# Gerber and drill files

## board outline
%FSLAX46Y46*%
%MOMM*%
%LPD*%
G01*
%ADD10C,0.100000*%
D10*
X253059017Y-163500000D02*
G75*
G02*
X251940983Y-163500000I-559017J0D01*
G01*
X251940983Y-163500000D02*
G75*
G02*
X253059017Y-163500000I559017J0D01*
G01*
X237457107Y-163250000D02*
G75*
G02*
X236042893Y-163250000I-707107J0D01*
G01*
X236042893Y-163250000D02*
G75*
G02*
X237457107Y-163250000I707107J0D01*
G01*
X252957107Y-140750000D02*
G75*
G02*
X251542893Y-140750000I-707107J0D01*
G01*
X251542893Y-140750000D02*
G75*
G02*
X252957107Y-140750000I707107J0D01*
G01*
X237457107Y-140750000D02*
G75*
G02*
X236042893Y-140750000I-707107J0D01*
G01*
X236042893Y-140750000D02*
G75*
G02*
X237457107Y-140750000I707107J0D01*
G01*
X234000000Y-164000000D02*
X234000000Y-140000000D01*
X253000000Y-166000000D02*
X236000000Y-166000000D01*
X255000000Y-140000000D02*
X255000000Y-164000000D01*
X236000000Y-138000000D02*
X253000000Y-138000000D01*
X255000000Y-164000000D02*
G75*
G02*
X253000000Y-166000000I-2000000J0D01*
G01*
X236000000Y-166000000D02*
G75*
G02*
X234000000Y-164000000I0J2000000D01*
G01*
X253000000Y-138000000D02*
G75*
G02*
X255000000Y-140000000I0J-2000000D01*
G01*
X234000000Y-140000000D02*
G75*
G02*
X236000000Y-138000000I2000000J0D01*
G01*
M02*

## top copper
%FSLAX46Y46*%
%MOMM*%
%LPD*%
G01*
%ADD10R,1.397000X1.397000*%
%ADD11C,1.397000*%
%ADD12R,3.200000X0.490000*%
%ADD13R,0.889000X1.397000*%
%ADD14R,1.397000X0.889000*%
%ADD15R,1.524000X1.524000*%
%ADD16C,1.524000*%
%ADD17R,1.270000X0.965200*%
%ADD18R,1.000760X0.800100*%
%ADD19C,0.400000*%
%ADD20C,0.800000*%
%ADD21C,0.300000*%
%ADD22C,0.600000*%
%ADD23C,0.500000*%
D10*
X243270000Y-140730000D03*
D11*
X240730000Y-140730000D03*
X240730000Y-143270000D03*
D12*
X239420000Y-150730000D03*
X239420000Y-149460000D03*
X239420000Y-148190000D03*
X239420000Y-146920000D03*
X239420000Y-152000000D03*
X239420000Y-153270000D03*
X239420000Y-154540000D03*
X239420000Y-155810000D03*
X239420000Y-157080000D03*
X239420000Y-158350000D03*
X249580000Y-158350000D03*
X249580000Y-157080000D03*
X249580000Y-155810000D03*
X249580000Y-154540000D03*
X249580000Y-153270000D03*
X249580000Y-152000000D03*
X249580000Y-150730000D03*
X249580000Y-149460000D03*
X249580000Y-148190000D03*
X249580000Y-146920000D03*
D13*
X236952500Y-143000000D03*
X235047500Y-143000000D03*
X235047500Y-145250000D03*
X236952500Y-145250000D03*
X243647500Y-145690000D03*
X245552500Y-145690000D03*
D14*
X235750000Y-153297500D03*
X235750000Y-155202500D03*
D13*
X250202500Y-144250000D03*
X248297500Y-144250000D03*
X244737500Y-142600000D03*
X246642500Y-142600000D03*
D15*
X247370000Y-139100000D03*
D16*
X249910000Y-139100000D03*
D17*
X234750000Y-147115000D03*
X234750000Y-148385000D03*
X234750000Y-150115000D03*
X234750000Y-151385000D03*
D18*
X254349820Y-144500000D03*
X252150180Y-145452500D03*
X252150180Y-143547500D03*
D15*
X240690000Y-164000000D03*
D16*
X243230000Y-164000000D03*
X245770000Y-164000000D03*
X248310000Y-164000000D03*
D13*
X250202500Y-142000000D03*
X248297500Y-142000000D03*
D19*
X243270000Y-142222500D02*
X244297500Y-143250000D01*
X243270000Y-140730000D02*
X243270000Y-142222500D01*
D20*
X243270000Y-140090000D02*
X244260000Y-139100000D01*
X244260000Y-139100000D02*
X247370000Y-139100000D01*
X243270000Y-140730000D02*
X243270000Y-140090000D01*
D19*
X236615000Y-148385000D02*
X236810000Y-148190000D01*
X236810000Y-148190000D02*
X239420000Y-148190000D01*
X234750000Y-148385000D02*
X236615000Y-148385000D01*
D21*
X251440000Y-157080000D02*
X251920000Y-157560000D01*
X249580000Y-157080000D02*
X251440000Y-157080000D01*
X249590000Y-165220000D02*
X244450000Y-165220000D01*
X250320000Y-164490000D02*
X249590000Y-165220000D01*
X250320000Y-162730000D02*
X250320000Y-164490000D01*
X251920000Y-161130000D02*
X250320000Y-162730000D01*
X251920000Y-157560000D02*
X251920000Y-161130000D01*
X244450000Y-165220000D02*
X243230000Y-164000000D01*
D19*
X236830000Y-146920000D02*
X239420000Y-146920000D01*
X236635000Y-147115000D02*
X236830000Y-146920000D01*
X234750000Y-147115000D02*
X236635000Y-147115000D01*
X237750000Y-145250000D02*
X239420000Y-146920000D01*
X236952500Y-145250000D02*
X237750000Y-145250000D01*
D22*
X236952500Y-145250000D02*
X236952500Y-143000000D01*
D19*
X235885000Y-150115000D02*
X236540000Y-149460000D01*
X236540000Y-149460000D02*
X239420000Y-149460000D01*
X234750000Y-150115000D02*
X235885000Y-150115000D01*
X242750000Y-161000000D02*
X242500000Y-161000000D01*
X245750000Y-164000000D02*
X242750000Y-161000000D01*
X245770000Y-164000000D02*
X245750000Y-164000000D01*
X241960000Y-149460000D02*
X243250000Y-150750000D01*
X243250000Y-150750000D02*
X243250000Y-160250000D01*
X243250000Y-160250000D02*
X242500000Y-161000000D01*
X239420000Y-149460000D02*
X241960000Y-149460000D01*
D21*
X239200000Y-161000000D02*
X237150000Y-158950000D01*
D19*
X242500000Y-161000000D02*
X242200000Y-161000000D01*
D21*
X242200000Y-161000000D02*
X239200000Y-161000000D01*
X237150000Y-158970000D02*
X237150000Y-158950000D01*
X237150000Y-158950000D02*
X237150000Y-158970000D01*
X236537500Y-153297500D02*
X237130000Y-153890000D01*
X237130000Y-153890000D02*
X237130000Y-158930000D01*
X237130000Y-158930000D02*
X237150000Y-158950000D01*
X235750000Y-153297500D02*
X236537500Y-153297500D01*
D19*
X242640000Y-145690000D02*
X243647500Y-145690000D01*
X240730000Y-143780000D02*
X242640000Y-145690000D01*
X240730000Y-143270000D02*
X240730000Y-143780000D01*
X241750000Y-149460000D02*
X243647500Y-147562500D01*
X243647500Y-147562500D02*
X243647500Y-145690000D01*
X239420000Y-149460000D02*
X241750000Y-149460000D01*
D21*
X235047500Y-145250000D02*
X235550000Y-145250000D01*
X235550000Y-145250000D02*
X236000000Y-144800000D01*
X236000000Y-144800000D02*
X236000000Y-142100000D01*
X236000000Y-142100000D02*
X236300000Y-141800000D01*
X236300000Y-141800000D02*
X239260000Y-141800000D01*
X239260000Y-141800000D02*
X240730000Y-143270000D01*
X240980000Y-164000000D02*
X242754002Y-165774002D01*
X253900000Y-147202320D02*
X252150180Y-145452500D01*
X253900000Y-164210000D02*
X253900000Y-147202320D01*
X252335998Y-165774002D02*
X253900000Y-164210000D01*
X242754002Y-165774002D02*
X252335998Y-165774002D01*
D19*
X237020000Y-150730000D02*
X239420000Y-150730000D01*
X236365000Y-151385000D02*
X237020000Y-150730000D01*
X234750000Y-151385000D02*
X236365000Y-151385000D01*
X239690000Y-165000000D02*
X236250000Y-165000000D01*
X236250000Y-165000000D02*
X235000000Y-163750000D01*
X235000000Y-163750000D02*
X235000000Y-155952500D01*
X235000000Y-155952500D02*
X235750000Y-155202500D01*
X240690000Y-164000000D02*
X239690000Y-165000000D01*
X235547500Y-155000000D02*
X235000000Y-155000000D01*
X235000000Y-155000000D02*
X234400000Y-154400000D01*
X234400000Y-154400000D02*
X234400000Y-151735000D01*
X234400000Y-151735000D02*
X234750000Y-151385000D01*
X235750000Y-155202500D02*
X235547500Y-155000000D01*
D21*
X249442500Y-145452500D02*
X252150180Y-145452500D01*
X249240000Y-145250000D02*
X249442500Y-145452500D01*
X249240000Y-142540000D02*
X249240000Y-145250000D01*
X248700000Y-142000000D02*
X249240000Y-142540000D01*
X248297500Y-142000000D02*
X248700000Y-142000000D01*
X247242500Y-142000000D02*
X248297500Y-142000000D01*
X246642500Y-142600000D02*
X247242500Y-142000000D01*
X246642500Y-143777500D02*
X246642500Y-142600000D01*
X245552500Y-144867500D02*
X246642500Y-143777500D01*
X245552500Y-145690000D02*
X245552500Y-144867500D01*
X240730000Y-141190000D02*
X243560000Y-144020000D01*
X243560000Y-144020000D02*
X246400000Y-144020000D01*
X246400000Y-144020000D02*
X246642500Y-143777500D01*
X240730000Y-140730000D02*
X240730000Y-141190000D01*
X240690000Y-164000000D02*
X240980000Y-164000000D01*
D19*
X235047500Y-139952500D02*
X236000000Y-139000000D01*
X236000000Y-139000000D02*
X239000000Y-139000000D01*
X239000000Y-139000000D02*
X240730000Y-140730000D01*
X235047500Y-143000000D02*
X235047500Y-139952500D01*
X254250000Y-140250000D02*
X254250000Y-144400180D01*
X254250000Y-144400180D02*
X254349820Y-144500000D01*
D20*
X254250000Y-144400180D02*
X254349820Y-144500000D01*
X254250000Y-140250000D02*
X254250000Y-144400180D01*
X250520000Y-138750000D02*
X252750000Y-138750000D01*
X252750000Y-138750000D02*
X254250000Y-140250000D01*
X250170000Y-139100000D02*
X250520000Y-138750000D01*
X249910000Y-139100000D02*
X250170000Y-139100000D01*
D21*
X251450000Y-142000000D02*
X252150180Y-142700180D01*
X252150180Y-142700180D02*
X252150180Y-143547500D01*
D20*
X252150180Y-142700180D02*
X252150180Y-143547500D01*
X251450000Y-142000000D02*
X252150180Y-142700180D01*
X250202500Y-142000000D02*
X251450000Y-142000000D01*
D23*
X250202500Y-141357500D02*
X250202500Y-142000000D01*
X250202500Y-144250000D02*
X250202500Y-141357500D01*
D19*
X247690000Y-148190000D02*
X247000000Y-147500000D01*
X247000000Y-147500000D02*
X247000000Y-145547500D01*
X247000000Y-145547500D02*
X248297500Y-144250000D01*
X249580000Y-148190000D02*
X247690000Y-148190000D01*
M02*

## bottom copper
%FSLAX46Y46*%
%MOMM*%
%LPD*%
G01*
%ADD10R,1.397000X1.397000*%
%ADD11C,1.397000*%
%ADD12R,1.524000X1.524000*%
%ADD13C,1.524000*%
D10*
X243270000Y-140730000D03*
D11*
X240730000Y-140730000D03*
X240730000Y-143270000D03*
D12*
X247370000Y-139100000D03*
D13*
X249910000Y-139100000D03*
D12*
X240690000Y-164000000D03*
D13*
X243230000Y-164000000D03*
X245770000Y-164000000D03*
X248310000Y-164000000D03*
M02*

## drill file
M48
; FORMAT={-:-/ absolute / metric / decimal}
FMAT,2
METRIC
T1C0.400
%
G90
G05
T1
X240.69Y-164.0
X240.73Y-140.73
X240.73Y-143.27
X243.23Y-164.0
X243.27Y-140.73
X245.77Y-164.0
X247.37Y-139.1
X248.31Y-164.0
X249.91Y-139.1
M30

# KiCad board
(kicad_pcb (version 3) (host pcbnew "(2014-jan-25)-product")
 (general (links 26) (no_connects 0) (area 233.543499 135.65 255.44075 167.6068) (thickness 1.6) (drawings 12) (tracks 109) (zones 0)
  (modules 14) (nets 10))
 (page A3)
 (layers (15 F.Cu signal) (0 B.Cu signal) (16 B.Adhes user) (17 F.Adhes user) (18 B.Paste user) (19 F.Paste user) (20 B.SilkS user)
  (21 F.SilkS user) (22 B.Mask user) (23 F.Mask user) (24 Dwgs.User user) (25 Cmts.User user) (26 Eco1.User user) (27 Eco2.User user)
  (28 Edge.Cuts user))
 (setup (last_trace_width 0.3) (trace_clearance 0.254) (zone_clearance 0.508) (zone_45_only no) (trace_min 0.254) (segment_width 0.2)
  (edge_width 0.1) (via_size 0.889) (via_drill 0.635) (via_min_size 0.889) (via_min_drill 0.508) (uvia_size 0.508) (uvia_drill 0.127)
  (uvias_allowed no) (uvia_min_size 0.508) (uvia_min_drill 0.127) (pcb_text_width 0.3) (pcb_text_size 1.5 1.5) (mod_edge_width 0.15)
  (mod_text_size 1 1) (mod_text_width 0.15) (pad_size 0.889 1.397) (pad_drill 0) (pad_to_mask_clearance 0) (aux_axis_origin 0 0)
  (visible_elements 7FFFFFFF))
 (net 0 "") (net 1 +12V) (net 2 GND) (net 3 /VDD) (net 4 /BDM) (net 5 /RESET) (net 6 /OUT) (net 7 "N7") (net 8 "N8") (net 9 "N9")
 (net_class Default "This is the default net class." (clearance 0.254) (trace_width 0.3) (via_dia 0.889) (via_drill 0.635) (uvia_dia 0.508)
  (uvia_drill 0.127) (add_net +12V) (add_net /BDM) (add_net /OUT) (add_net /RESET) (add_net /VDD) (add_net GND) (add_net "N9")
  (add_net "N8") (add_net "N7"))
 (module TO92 (layer F.Cu) (at 242 142)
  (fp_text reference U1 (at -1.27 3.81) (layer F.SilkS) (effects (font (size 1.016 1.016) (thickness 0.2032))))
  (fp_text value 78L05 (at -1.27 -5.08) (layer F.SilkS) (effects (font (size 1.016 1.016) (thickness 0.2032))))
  (pad 1 thru_hole rect (at 1.27 -1.27) (size 1.397 1.397) (drill 0.4) (layers *.Cu *.Mask F.SilkS) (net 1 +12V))
  (pad 2 thru_hole circle (at -1.27 -1.27) (size 1.397 1.397) (drill 0.4) (layers *.Cu *.Mask F.SilkS) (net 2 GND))
  (pad 3 thru_hole circle (at -1.27 1.27) (size 1.397 1.397) (drill 0.4) (layers *.Cu *.Mask F.SilkS) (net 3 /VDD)))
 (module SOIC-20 (layer F.Cu) (at 244.5 152)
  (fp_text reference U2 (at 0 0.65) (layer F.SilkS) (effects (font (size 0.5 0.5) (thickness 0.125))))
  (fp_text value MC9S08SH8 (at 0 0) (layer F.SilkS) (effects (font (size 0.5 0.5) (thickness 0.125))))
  (pad 4 smd rect (at -5.08 -1.27) (size 3.2 0.49) (layers F.Cu F.Paste F.Mask) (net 2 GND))
  (pad 3 smd rect (at -5.08 -2.54) (size 3.2 0.49) (layers F.Cu F.Paste F.Mask) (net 3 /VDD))
  (pad 2 smd rect (at -5.08 -3.81) (size 3.2 0.49) (layers F.Cu F.Paste F.Mask) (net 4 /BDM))
  (pad 1 smd rect (at -5.08 -5.08) (size 3.2 0.49) (layers F.Cu F.Paste F.Mask) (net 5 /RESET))
  (pad 5 smd rect (at -5.08 0) (size 3.2 0.49) (layers F.Cu F.Paste F.Mask))
  (pad 6 smd rect (at -5.08 1.27) (size 3.2 0.49) (layers F.Cu F.Paste F.Mask))
  (pad 7 smd rect (at -5.08 2.54) (size 3.2 0.49) (layers F.Cu F.Paste F.Mask))
  (pad 8 smd rect (at -5.08 3.81) (size 3.2 0.49) (layers F.Cu F.Paste F.Mask))
  (pad 9 smd rect (at -5.08 5.08) (size 3.2 0.49) (layers F.Cu F.Paste F.Mask))
  (pad 10 smd rect (at -5.08 6.35) (size 3.2 0.49) (layers F.Cu F.Paste F.Mask))
  (pad 11 smd rect (at 5.08 6.35) (size 3.2 0.49) (layers F.Cu F.Paste F.Mask))
  (pad 12 smd rect (at 5.08 5.08) (size 3.2 0.49) (layers F.Cu F.Paste F.Mask) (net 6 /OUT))
  (pad 13 smd rect (at 5.08 3.81) (size 3.2 0.49) (layers F.Cu F.Paste F.Mask))
  (pad 14 smd rect (at 5.08 2.54) (size 3.2 0.49) (layers F.Cu F.Paste F.Mask))
  (pad 15 smd rect (at 5.08 1.27) (size 3.2 0.49) (layers F.Cu F.Paste F.Mask))
  (pad 16 smd rect (at 5.08 0) (size 3.2 0.49) (layers F.Cu F.Paste F.Mask))
  (pad 17 smd rect (at 5.08 -1.27) (size 3.2 0.49) (layers F.Cu F.Paste F.Mask))
  (pad 18 smd rect (at 5.08 -2.54) (size 3.2 0.49) (layers F.Cu F.Paste F.Mask))
  (pad 19 smd rect (at 5.08 -3.81) (size 3.2 0.49) (layers F.Cu F.Paste F.Mask) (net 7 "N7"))
  (pad 20 smd rect (at 5.08 -5.08) (size 3.2 0.49) (layers F.Cu F.Paste F.Mask)))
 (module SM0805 (layer F.Cu) (at 236 143 180)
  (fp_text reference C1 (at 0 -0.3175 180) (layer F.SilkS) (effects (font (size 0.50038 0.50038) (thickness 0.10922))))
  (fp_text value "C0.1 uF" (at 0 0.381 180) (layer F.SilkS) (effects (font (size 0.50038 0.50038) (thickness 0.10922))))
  (pad 1 smd rect (at -0.9525 0 180) (size 0.889 1.397) (layers F.Cu F.Paste F.Mask) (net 5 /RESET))
  (pad 2 smd rect (at 0.9525 0 180) (size 0.889 1.397) (layers F.Cu F.Paste F.Mask) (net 2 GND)))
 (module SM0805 (layer F.Cu) (at 236 145.25)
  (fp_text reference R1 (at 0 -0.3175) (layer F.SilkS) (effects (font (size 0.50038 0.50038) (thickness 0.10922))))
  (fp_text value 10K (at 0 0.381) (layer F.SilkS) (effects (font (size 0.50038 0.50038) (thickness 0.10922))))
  (pad 1 smd rect (at -0.9525 0) (size 0.889 1.397) (layers F.Cu F.Paste F.Mask) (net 3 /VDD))
  (pad 2 smd rect (at 0.9525 0) (size 0.889 1.397) (layers F.Cu F.Paste F.Mask) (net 5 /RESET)))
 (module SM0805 (layer F.Cu) (at 244.6 145.69)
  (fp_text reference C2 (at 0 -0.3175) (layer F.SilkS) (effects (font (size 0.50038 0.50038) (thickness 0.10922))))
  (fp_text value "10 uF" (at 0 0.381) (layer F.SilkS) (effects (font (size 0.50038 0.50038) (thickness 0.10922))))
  (pad 1 smd rect (at -0.9525 0) (size 0.889 1.397) (layers F.Cu F.Paste F.Mask) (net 3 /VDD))
  (pad 2 smd rect (at 0.9525 0) (size 0.889 1.397) (layers F.Cu F.Paste F.Mask) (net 2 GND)))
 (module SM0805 (layer F.Cu) (at 235.75 154.25 270)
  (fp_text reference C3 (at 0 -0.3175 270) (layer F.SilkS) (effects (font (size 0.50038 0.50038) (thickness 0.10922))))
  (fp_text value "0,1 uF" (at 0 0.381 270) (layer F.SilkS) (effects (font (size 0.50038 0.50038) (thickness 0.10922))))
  (pad 1 smd rect (at -0.9525 0 270) (size 0.889 1.397) (layers F.Cu F.Paste F.Mask) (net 3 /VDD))
  (pad 2 smd rect (at 0.9525 0 270) (size 0.889 1.397) (layers F.Cu F.Paste F.Mask) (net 2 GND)))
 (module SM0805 (layer F.Cu) (at 249.25 144.25 180)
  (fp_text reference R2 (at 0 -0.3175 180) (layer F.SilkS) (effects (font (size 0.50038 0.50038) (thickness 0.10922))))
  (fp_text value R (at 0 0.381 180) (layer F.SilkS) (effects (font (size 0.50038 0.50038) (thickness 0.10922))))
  (pad 1 smd rect (at -0.9525 0 180) (size 0.889 1.397) (layers F.Cu F.Paste F.Mask) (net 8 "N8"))
  (pad 2 smd rect (at 0.9525 0 180) (size 0.889 1.397) (layers F.Cu F.Paste F.Mask) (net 7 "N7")))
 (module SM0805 (layer F.Cu) (at 245.69 142.6)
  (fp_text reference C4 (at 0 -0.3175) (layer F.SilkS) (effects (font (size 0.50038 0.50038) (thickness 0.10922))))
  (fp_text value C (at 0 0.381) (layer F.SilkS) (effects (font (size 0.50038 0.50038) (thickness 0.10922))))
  (pad 1 smd rect (at -0.9525 0) (size 0.889 1.397) (layers F.Cu F.Paste F.Mask) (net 1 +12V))
  (pad 2 smd rect (at 0.9525 0) (size 0.889 1.397) (layers F.Cu F.Paste F.Mask) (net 2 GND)))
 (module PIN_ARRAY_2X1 (layer F.Cu) (at 248.64 139.1)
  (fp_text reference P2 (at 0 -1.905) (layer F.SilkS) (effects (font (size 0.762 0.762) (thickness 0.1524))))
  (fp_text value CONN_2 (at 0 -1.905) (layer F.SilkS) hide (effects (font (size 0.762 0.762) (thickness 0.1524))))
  (pad 1 thru_hole rect (at -1.27 0) (size 1.524 1.524) (drill 0.4) (layers *.Cu *.Mask F.SilkS) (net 1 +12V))
  (pad 2 thru_hole circle (at 1.27 0) (size 1.524 1.524) (drill 0.4) (layers *.Cu *.Mask F.SilkS) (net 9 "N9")))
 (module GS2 (layer F.Cu) (at 234.75 147.75)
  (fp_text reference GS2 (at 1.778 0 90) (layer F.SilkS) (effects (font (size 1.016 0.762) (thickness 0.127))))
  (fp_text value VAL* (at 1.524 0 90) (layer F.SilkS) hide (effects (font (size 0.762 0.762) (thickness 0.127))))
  (pad 1 smd rect (at 0 -0.635) (size 1.27 0.9652) (layers F.Cu F.Paste F.Mask) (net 5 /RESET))
  (pad 2 smd rect (at 0 0.635) (size 1.27 0.9652) (layers F.Cu F.Paste F.Mask) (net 4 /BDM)))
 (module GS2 (layer F.Cu) (at 234.75 150.75)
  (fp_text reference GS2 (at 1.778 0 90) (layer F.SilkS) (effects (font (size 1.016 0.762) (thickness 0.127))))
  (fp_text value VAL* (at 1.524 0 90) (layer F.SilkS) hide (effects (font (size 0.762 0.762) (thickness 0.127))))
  (pad 1 smd rect (at 0 -0.635) (size 1.27 0.9652) (layers F.Cu F.Paste F.Mask) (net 3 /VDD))
  (pad 2 smd rect (at 0 0.635) (size 1.27 0.9652) (layers F.Cu F.Paste F.Mask) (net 2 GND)))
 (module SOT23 (layer F.Cu) (at 253.25 144.5 270)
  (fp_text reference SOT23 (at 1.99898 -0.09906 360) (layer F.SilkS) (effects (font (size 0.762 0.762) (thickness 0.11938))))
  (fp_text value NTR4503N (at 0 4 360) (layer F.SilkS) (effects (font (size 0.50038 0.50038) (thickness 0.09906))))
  (pad 3 smd rect (at 0 -1.09982 270) (size 0.8001 1.00076) (layers F.Cu F.Paste F.Mask) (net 9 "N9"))
  (pad 2 smd rect (at 0.9525 1.09982 270) (size 0.8001 1.00076) (layers F.Cu F.Paste F.Mask) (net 2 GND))
  (pad 1 smd rect (at -0.9525 1.09982 270) (size 0.8001 1.00076) (layers F.Cu F.Paste F.Mask) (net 8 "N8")))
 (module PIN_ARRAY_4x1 (layer F.Cu) (at 244.5 164)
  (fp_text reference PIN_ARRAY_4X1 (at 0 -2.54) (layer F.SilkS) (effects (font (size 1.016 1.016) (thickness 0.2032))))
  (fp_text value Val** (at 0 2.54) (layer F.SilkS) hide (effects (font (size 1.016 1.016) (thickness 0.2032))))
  (pad 1 thru_hole rect (at -3.81 0) (size 1.524 1.524) (drill 0.4) (layers *.Cu *.Mask F.SilkS) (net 2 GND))
  (pad 2 thru_hole circle (at -1.27 0) (size 1.524 1.524) (drill 0.4) (layers *.Cu *.Mask F.SilkS) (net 6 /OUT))
  (pad 3 thru_hole circle (at 1.27 0) (size 1.524 1.524) (drill 0.4) (layers *.Cu *.Mask F.SilkS) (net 3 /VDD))
  (pad 4 thru_hole circle (at 3.81 0) (size 1.524 1.524) (drill 0.4) (layers *.Cu *.Mask F.SilkS)))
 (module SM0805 (layer F.Cu) (at 249.25 142 180)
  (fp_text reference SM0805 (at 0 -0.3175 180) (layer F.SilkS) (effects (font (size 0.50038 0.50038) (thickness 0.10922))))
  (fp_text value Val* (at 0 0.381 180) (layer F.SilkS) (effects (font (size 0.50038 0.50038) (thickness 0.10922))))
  (pad 1 smd rect (at -0.9525 0 180) (size 0.889 1.397) (layers F.Cu F.Paste F.Mask) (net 8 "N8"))
  (pad 2 smd rect (at 0.9525 0 180) (size 0.889 1.397) (layers F.Cu F.Paste F.Mask) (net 2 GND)))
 (gr_circle (center 252.5 163.5) (end 253 163.75) (layer Edge.Cuts) (width 0.1))
 (gr_circle (center 236.75 163.25) (end 237.25 163.75) (layer Edge.Cuts) (width 0.1))
 (gr_circle (center 252.25 140.75) (end 252.75 140.25) (layer Edge.Cuts) (width 0.1))
 (gr_circle (center 236.75 140.75) (end 236.25 140.25) (layer Edge.Cuts) (width 0.1))
 (gr_line (start 234 164) (end 234 140) (angle 90) (layer Edge.Cuts) (width 0.1))
 (gr_line (start 253 166) (end 236 166) (angle 90) (layer Edge.Cuts) (width 0.1))
 (gr_line (start 255 140) (end 255 164) (angle 90) (layer Edge.Cuts) (width 0.1))
 (gr_line (start 236 138) (end 253 138) (angle 90) (layer Edge.Cuts) (width 0.1))
 (gr_arc (start 253 164) (end 255 164) (angle 90) (layer Edge.Cuts) (width 0.1))
 (gr_arc (start 236 164) (end 236 166) (angle 90) (layer Edge.Cuts) (width 0.1))
 (gr_arc (start 253 140) (end 253 138) (angle 90) (layer Edge.Cuts) (width 0.1))
 (gr_arc (start 236 140) (end 234 140) (angle 90) (layer Edge.Cuts) (width 0.1))
 (segment (start 243.27 142.2225) (end 244.2975 143.25) (width 0.4) (layer F.Cu) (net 1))
 (segment (start 243.27 140.73) (end 243.27 142.2225) (width 0.4) (layer F.Cu) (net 1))
 (segment (start 243.27 140.09) (end 244.26 139.1) (width 0.8) (layer F.Cu) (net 1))
 (segment (start 244.26 139.1) (end 247.37 139.1) (width 0.8) (layer F.Cu) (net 1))
 (segment (start 243.27 140.73) (end 243.27 140.09) (width 0.8) (layer F.Cu) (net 1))
 (segment (start 236.615 148.385) (end 236.81 148.19) (width 0.4) (layer F.Cu) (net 4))
 (segment (start 236.81 148.19) (end 239.42 148.19) (width 0.4) (layer F.Cu) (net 4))
 (segment (start 234.75 148.385) (end 236.615 148.385) (width 0.4) (layer F.Cu) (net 4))
 (segment (start 251.44 157.08) (end 251.92 157.56) (width 0.3) (layer F.Cu) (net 6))
 (segment (start 249.58 157.08) (end 251.44 157.08) (width 0.3) (layer F.Cu) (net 6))
 (segment (start 249.59 165.22) (end 244.45 165.22) (width 0.3) (layer F.Cu) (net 6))
 (segment (start 250.32 164.49) (end 249.59 165.22) (width 0.3) (layer F.Cu) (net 6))
 (segment (start 250.32 162.73) (end 250.32 164.49) (width 0.3) (layer F.Cu) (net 6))
 (segment (start 251.92 161.13) (end 250.32 162.73) (width 0.3) (layer F.Cu) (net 6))
 (segment (start 251.92 157.56) (end 251.92 161.13) (width 0.3) (layer F.Cu) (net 6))
 (segment (start 244.45 165.22) (end 243.23 164) (width 0.3) (layer F.Cu) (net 6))
 (segment (start 236.83 146.92) (end 239.42 146.92) (width 0.4) (layer F.Cu) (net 5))
 (segment (start 236.635 147.115) (end 236.83 146.92) (width 0.4) (layer F.Cu) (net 5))
 (segment (start 234.75 147.115) (end 236.635 147.115) (width 0.4) (layer F.Cu) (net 5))
 (segment (start 237.75 145.25) (end 239.42 146.92) (width 0.4) (layer F.Cu) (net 5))
 (segment (start 236.9525 145.25) (end 237.75 145.25) (width 0.4) (layer F.Cu) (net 5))
 (segment (start 236.9525 145.25) (end 236.9525 143) (width 0.6) (layer F.Cu) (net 5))
 (segment (start 235.885 150.115) (end 236.54 149.46) (width 0.4) (layer F.Cu) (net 3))
 (segment (start 236.54 149.46) (end 239.42 149.46) (width 0.4) (layer F.Cu) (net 3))
 (segment (start 234.75 150.115) (end 235.885 150.115) (width 0.4) (layer F.Cu) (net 3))
 (segment (start 242.75 161) (end 242.5 161) (width 0.4) (layer F.Cu) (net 3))
 (segment (start 245.75 164) (end 242.75 161) (width 0.4) (layer F.Cu) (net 3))
 (segment (start 245.77 164) (end 245.75 164) (width 0.4) (layer F.Cu) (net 3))
 (segment (start 241.96 149.46) (end 243.25 150.75) (width 0.4) (layer F.Cu) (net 3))
 (segment (start 243.25 150.75) (end 243.25 160.25) (width 0.4) (layer F.Cu) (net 3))
 (segment (start 243.25 160.25) (end 242.5 161) (width 0.4) (layer F.Cu) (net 3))
 (segment (start 239.42 149.46) (end 241.96 149.46) (width 0.4) (layer F.Cu) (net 3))
 (segment (start 239.2 161) (end 237.15 158.95) (width 0.3) (layer F.Cu) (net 3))
 (segment (start 242.5 161) (end 242.2 161) (width 0.4) (layer F.Cu) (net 3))
 (segment (start 242.2 161) (end 239.2 161) (width 0.3) (layer F.Cu) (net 3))
 (segment (start 237.15 158.97) (end 237.15 158.95) (width 0.3) (layer F.Cu) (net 3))
 (segment (start 237.15 158.95) (end 237.15 158.97) (width 0.3) (layer F.Cu) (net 3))
 (segment (start 236.5375 153.2975) (end 237.13 153.89) (width 0.3) (layer F.Cu) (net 3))
 (segment (start 237.13 153.89) (end 237.13 158.93) (width 0.3) (layer F.Cu) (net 3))
 (segment (start 237.13 158.93) (end 237.15 158.95) (width 0.3) (layer F.Cu) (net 3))
 (segment (start 235.75 153.2975) (end 236.5375 153.2975) (width 0.3) (layer F.Cu) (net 3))
 (segment (start 242.64 145.69) (end 243.6475 145.69) (width 0.4) (layer F.Cu) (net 3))
 (segment (start 240.73 143.78) (end 242.64 145.69) (width 0.4) (layer F.Cu) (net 3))
 (segment (start 240.73 143.27) (end 240.73 143.78) (width 0.4) (layer F.Cu) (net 3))
 (segment (start 241.75 149.46) (end 243.6475 147.5625) (width 0.4) (layer F.Cu) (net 3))
 (segment (start 243.6475 147.5625) (end 243.6475 145.69) (width 0.4) (layer F.Cu) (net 3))
 (segment (start 239.42 149.46) (end 241.75 149.46) (width 0.4) (layer F.Cu) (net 3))
 (segment (start 235.0475 145.25) (end 235.55 145.25) (width 0.3) (layer F.Cu) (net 3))
 (segment (start 235.55 145.25) (end 236 144.8) (width 0.3) (layer F.Cu) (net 3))
 (segment (start 236 144.8) (end 236 142.1) (width 0.3) (layer F.Cu) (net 3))
 (segment (start 236 142.1) (end 236.3 141.8) (width 0.3) (layer F.Cu) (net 3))
 (segment (start 236.3 141.8) (end 239.26 141.8) (width 0.3) (layer F.Cu) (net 3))
 (segment (start 239.26 141.8) (end 240.73 143.27) (width 0.3) (layer F.Cu) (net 3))
 (segment (start 240.98 164) (end 242.754002 165.774002) (width 0.3) (layer F.Cu) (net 2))
 (segment (start 253.9 147.20232) (end 252.15018 145.4525) (width 0.3) (layer F.Cu) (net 2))
 (segment (start 253.9 164.21) (end 253.9 147.20232) (width 0.3) (layer F.Cu) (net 2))
 (segment (start 252.335998 165.774002) (end 253.9 164.21) (width 0.3) (layer F.Cu) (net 2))
 (segment (start 242.754002 165.774002) (end 252.335998 165.774002) (width 0.3) (layer F.Cu) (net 2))
 (segment (start 237.02 150.73) (end 239.42 150.73) (width 0.4) (layer F.Cu) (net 2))
 (segment (start 236.365 151.385) (end 237.02 150.73) (width 0.4) (layer F.Cu) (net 2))
 (segment (start 234.75 151.385) (end 236.365 151.385) (width 0.4) (layer F.Cu) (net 2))
 (segment (start 239.69 165) (end 236.25 165) (width 0.4) (layer F.Cu) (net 2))
 (segment (start 236.25 165) (end 235 163.75) (width 0.4) (layer F.Cu) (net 2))
 (segment (start 235 163.75) (end 235 155.9525) (width 0.4) (layer F.Cu) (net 2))
 (segment (start 235 155.9525) (end 235.75 155.2025) (width 0.4) (layer F.Cu) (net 2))
 (segment (start 240.69 164) (end 239.69 165) (width 0.4) (layer F.Cu) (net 2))
 (segment (start 235.5475 155) (end 235 155) (width 0.4) (layer F.Cu) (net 2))
 (segment (start 235 155) (end 234.4 154.4) (width 0.4) (layer F.Cu) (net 2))
 (segment (start 234.4 154.4) (end 234.4 151.735) (width 0.4) (layer F.Cu) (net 2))
 (segment (start 234.4 151.735) (end 234.75 151.385) (width 0.4) (layer F.Cu) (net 2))
 (segment (start 235.75 155.2025) (end 235.5475 155) (width 0.4) (layer F.Cu) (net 2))
 (segment (start 249.4425 145.4525) (end 252.15018 145.4525) (width 0.3) (layer F.Cu) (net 2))
 (segment (start 249.24 145.25) (end 249.4425 145.4525) (width 0.3) (layer F.Cu) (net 2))
 (segment (start 249.24 142.54) (end 249.24 145.25) (width 0.3) (layer F.Cu) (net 2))
 (segment (start 248.7 142) (end 249.24 142.54) (width 0.3) (layer F.Cu) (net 2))
 (segment (start 248.2975 142) (end 248.7 142) (width 0.3) (layer F.Cu) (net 2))
 (segment (start 247.2425 142) (end 248.2975 142) (width 0.3) (layer F.Cu) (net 2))
 (segment (start 246.6425 142.6) (end 247.2425 142) (width 0.3) (layer F.Cu) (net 2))
 (segment (start 246.6425 143.7775) (end 246.6425 142.6) (width 0.3) (layer F.Cu) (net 2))
 (segment (start 245.5525 144.8675) (end 246.6425 143.7775) (width 0.3) (layer F.Cu) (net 2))
 (segment (start 245.5525 145.69) (end 245.5525 144.8675) (width 0.3) (layer F.Cu) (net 2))
 (segment (start 240.73 141.19) (end 243.56 144.02) (width 0.3) (layer F.Cu) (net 2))
 (segment (start 243.56 144.02) (end 246.4 144.02) (width 0.3) (layer F.Cu) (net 2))
 (segment (start 246.4 144.02) (end 246.6425 143.7775) (width 0.3) (layer F.Cu) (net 2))
 (segment (start 240.73 140.73) (end 240.73 141.19) (width 0.3) (layer F.Cu) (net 2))
 (segment (start 240.69 164) (end 240.98 164) (width 0.3) (layer F.Cu) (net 2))
 (segment (start 235.0475 139.9525) (end 236 139) (width 0.4) (layer F.Cu) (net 2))
 (segment (start 236 139) (end 239 139) (width 0.4) (layer F.Cu) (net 2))
 (segment (start 239 139) (end 240.73 140.73) (width 0.4) (layer F.Cu) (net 2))
 (segment (start 235.0475 143) (end 235.0475 139.9525) (width 0.4) (layer F.Cu) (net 2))
 (segment (start 254.25 140.25) (end 254.25 144.40018) (width 0.4) (layer F.Cu) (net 9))
 (segment (start 254.25 144.40018) (end 254.34982 144.5) (width 0.4) (layer F.Cu) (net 9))
 (segment (start 254.25 144.40018) (end 254.34982 144.5) (width 0.8) (layer F.Cu) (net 9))
 (segment (start 254.25 140.25) (end 254.25 144.40018) (width 0.8) (layer F.Cu) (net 9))
 (segment (start 250.52 138.75) (end 252.75 138.75) (width 0.8) (layer F.Cu) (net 9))
 (segment (start 252.75 138.75) (end 254.25 140.25) (width 0.8) (layer F.Cu) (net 9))
 (segment (start 250.17 139.1) (end 250.52 138.75) (width 0.8) (layer F.Cu) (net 9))
 (segment (start 249.91 139.1) (end 250.17 139.1) (width 0.8) (layer F.Cu) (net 9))
 (segment (start 251.45 142) (end 252.15018 142.70018) (width 0.3) (layer F.Cu) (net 8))
 (segment (start 252.15018 142.70018) (end 252.15018 143.5475) (width 0.3) (layer F.Cu) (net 8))
 (segment (start 252.15018 142.70018) (end 252.15018 143.5475) (width 0.8) (layer F.Cu) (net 8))
 (segment (start 251.45 142) (end 252.15018 142.70018) (width 0.8) (layer F.Cu) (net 8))
 (segment (start 250.2025 142) (end 251.45 142) (width 0.8) (layer F.Cu) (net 8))
 (segment (start 250.2025 141.3575) (end 250.2025 142) (width 0.5) (layer F.Cu) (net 8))
 (segment (start 250.2025 144.25) (end 250.2025 141.3575) (width 0.5) (layer F.Cu) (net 8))
 (segment (start 247.69 148.19) (end 247 147.5) (width 0.4) (layer F.Cu) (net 7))
 (segment (start 247 147.5) (end 247 145.5475) (width 0.4) (layer F.Cu) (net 7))
 (segment (start 247 145.5475) (end 248.2975 144.25) (width 0.4) (layer F.Cu) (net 7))
 (segment (start 249.58 148.19) (end 247.69 148.19) (width 0.4) (layer F.Cu) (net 7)))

